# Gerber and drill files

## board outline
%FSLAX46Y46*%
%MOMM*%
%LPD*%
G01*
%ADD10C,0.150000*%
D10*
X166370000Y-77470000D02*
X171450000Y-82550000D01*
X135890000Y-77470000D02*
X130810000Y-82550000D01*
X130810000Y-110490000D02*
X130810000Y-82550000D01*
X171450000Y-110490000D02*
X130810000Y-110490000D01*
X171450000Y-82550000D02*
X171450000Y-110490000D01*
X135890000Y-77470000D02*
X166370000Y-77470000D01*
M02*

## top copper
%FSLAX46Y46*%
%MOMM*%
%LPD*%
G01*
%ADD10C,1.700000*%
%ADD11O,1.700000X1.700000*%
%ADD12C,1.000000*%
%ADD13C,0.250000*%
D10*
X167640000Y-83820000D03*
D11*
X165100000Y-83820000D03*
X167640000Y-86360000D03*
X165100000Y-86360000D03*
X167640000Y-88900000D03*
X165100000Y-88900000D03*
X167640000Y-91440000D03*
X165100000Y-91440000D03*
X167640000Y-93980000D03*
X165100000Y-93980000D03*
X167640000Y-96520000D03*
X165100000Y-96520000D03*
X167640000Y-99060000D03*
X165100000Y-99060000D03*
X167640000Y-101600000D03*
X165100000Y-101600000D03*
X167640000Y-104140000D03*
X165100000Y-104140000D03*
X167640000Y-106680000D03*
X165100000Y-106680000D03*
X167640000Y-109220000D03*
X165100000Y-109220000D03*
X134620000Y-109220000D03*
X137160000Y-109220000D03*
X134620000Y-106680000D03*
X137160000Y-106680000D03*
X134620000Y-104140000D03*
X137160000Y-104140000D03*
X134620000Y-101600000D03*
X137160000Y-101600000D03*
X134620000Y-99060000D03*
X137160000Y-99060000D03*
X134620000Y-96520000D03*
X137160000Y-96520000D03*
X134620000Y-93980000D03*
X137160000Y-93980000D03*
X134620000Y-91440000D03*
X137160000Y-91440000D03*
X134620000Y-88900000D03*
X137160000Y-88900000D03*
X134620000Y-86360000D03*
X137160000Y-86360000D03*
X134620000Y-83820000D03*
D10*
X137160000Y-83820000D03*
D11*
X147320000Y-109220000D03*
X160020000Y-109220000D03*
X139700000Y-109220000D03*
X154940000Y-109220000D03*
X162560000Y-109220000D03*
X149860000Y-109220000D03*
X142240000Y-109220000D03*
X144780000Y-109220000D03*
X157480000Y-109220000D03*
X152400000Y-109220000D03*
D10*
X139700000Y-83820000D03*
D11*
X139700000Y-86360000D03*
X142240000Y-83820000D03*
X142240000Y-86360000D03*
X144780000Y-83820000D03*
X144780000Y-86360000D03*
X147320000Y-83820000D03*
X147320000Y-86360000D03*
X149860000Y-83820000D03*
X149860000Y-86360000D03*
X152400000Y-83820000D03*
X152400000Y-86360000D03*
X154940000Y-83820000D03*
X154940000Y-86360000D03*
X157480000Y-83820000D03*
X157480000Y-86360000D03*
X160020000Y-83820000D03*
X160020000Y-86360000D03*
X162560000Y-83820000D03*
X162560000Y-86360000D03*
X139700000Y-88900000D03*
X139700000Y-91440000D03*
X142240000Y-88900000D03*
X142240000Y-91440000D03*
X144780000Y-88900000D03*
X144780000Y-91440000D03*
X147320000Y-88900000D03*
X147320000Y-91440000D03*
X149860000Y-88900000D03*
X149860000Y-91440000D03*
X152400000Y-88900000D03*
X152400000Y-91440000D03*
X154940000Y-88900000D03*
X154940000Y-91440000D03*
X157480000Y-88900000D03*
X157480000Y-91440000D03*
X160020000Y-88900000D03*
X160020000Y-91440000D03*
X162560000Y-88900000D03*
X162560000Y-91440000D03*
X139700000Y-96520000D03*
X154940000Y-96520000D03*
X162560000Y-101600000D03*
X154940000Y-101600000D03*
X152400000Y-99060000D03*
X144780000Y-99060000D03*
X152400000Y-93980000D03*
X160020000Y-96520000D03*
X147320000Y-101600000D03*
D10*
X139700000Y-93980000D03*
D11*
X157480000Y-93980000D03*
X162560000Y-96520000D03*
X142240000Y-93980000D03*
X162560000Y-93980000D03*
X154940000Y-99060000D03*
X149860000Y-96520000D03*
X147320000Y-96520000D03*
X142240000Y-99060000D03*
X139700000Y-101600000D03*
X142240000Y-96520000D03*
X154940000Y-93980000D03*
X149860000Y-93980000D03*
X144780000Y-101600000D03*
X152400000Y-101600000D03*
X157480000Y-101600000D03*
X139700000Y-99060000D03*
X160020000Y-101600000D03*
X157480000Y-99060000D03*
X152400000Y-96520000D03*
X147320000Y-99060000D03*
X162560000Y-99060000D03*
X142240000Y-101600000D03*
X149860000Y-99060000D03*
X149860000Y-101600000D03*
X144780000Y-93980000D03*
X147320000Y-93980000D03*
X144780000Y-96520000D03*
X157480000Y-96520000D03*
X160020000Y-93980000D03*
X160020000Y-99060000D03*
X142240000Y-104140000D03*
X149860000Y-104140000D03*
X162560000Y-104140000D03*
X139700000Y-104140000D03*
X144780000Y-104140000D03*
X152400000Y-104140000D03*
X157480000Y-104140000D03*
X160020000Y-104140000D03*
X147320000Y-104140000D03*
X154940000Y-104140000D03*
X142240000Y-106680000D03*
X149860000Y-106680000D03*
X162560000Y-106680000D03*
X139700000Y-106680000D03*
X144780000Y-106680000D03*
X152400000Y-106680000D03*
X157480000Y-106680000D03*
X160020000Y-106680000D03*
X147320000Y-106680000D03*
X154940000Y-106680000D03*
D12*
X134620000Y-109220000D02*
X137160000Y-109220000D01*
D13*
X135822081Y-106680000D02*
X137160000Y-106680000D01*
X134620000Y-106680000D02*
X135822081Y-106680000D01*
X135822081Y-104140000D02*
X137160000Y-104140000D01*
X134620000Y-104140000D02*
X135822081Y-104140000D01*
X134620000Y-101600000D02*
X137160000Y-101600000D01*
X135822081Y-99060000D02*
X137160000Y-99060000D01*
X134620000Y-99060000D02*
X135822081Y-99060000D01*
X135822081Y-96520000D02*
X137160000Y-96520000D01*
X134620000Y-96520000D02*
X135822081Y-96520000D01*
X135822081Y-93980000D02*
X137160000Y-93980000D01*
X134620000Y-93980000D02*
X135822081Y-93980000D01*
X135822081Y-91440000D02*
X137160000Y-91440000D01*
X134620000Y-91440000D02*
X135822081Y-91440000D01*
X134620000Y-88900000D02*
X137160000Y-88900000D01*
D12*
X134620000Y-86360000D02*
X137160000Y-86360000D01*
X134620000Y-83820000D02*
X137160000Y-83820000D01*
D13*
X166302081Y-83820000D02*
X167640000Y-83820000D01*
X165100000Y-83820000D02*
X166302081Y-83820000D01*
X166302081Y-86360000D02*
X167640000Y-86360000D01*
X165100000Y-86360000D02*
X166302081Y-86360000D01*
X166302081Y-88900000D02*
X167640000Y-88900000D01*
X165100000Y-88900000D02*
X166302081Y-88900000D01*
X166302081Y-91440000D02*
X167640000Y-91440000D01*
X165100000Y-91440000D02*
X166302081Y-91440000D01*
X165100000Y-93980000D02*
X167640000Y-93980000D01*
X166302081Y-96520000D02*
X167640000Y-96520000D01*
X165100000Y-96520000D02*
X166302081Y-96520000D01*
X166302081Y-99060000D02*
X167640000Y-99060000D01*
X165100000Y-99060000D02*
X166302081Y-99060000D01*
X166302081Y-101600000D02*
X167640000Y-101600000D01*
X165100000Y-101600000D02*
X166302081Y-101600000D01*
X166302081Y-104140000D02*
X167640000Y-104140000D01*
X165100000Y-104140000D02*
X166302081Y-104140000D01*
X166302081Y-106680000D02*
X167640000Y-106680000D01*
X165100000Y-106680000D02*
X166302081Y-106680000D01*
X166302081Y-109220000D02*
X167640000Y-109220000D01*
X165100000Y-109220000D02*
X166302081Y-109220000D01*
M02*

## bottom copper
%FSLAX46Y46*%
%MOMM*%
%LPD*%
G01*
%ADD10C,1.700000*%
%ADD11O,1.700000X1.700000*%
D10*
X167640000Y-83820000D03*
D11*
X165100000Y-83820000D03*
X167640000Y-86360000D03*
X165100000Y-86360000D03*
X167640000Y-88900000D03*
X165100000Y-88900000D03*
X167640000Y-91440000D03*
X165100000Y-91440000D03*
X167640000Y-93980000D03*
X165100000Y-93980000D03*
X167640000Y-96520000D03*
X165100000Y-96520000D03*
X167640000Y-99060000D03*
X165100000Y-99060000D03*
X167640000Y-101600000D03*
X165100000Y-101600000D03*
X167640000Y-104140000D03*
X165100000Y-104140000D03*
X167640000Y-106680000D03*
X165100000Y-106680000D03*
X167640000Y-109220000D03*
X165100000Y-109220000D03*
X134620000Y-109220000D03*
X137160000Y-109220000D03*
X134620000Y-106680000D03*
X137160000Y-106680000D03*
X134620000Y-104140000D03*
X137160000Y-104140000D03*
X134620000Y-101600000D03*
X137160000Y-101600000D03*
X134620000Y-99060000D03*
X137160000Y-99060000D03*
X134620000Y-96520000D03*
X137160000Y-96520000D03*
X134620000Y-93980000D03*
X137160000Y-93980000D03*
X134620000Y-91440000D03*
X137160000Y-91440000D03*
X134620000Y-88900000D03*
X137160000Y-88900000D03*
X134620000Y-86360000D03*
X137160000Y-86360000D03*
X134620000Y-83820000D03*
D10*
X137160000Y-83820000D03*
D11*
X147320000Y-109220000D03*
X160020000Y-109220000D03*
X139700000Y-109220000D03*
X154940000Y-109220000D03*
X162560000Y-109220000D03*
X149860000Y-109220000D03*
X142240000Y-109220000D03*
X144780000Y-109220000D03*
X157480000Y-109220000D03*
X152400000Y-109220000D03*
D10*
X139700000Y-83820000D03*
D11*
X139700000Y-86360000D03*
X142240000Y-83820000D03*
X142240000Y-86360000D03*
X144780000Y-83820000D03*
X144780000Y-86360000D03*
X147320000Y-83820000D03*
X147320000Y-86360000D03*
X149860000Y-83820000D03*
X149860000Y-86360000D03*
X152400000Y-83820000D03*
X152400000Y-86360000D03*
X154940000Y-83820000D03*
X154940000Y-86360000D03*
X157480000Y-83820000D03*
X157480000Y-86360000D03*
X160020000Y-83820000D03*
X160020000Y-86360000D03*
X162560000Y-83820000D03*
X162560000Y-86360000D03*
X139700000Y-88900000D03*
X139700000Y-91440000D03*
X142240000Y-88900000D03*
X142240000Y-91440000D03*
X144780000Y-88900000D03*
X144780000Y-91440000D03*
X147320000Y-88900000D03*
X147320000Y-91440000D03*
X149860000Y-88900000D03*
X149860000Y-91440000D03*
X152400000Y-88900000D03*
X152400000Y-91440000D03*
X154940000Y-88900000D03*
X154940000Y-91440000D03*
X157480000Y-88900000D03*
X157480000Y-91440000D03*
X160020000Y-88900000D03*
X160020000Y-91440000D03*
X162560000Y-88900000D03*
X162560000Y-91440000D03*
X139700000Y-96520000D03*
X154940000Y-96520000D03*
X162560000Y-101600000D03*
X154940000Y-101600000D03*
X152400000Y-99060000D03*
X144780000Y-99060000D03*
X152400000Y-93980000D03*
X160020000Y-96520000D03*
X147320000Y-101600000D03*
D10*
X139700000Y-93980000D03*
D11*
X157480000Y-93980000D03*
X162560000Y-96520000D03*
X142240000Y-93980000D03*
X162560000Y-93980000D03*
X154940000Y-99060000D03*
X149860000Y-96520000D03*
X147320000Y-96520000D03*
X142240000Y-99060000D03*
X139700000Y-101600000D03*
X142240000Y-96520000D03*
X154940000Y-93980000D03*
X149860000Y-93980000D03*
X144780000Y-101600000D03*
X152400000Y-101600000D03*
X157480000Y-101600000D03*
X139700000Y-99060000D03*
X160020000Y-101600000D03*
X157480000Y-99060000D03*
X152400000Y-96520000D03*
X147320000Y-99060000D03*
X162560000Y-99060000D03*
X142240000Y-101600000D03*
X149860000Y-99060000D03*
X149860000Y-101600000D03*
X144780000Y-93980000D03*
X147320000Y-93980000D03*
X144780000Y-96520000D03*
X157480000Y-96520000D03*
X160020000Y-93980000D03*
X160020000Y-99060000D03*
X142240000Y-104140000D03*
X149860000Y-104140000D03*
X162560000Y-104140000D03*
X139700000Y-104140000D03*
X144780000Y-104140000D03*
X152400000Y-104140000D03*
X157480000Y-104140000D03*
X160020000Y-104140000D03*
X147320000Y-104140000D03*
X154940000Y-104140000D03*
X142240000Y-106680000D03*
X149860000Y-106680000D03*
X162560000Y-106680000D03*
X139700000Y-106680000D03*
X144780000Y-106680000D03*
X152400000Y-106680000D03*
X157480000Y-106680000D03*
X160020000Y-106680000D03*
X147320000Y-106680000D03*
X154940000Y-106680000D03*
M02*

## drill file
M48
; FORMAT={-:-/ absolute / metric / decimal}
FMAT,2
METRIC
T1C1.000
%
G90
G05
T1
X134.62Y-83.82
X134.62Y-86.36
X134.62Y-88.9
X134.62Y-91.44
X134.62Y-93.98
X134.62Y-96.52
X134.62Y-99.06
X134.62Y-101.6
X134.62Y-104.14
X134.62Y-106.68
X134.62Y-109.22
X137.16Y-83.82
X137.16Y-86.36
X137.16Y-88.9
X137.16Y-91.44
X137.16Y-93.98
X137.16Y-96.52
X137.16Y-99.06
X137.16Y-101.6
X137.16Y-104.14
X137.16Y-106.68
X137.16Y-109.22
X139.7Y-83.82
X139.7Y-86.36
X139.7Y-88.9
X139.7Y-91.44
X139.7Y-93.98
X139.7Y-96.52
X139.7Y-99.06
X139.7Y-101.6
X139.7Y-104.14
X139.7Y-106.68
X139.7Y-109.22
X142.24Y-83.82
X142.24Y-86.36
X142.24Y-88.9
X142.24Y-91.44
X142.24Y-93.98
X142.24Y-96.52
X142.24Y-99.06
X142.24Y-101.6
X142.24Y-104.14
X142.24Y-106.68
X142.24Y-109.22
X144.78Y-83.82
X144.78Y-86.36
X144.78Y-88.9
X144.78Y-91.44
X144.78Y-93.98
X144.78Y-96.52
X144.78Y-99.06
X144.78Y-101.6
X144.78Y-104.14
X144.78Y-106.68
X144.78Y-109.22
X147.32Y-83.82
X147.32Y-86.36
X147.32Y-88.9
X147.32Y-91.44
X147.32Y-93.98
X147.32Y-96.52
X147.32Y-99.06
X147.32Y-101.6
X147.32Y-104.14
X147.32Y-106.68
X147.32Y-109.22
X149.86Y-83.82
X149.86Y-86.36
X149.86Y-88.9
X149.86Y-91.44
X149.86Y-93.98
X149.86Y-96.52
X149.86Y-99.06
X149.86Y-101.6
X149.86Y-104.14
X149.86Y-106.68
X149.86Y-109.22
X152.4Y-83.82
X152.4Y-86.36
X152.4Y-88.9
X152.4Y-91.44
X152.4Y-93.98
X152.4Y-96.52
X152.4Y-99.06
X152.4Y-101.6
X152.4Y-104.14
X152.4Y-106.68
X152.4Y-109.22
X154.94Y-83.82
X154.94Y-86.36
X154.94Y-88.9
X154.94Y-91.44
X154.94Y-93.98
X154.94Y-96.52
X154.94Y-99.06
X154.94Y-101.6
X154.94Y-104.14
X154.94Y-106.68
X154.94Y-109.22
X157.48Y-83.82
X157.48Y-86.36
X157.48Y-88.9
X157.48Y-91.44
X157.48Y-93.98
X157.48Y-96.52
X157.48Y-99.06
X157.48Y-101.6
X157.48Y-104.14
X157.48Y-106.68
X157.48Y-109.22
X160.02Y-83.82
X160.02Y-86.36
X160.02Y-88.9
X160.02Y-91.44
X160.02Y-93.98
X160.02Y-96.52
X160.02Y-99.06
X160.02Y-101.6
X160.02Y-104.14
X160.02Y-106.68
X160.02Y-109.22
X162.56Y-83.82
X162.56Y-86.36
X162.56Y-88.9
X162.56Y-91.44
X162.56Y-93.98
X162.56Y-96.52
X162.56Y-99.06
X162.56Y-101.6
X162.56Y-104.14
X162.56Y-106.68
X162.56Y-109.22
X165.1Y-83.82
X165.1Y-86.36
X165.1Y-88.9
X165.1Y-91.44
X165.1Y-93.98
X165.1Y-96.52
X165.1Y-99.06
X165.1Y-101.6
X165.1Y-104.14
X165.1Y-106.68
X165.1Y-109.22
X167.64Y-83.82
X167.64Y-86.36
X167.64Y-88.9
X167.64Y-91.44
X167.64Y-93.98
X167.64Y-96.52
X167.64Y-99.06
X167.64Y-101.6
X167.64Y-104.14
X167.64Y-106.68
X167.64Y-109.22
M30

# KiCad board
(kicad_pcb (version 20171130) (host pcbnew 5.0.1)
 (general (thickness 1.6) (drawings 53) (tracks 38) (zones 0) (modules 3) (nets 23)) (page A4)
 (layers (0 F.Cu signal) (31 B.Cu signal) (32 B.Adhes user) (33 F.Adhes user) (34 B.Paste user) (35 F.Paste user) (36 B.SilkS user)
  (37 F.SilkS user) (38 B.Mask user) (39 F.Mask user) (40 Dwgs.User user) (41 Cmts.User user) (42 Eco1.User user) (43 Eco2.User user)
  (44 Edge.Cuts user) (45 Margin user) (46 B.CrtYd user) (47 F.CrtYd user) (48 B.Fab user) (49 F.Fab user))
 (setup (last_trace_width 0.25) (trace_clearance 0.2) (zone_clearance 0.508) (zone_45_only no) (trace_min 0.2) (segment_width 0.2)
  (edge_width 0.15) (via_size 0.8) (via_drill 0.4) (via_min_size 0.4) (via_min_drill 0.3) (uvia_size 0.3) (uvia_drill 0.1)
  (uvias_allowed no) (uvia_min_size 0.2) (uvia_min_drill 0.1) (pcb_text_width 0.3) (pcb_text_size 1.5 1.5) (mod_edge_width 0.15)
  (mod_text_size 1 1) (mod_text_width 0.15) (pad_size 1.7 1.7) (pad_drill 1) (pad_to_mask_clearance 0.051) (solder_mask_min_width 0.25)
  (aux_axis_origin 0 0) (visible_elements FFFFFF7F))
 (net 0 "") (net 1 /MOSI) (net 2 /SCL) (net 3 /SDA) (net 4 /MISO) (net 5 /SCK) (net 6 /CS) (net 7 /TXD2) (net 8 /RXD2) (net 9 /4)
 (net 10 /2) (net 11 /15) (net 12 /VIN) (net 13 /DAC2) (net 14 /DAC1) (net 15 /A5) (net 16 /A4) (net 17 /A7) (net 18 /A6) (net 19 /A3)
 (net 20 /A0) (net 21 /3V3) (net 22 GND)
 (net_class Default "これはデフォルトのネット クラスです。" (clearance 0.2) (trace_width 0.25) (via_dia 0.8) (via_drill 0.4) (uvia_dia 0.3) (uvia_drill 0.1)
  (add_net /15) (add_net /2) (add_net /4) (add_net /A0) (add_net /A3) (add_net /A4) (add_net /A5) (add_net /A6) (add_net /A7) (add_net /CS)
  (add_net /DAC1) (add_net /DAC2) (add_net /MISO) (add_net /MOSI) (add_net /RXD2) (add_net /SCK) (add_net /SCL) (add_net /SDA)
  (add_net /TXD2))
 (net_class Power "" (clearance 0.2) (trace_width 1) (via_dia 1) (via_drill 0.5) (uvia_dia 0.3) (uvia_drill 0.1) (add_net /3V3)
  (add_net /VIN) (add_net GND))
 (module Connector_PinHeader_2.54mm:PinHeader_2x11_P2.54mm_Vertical (layer B.Cu) (at 167.64 83.82 180)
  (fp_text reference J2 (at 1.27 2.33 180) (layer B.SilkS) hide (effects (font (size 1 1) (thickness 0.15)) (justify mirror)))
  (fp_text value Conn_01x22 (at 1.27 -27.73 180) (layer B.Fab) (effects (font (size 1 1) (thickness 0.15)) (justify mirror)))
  (pad 1 thru_hole circle (at 0 0 180) (size 1.7 1.7) (drill 1) (layers *.Cu *.Mask) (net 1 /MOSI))
  (pad 2 thru_hole oval (at 2.54 0 180) (size 1.7 1.7) (drill 1) (layers *.Cu *.Mask) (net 1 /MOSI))
  (pad 3 thru_hole oval (at 0 -2.54 180) (size 1.7 1.7) (drill 1) (layers *.Cu *.Mask) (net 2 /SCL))
  (pad 4 thru_hole oval (at 2.54 -2.54 180) (size 1.7 1.7) (drill 1) (layers *.Cu *.Mask) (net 2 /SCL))
  (pad 5 thru_hole oval (at 0 -5.08 180) (size 1.7 1.7) (drill 1) (layers *.Cu *.Mask) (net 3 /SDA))
  (pad 6 thru_hole oval (at 2.54 -5.08 180) (size 1.7 1.7) (drill 1) (layers *.Cu *.Mask) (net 3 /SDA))
  (pad 7 thru_hole oval (at 0 -7.62 180) (size 1.7 1.7) (drill 1) (layers *.Cu *.Mask) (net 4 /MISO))
  (pad 8 thru_hole oval (at 2.54 -7.62 180) (size 1.7 1.7) (drill 1) (layers *.Cu *.Mask) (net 4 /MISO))
  (pad 9 thru_hole oval (at 0 -10.16 180) (size 1.7 1.7) (drill 1) (layers *.Cu *.Mask) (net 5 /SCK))
  (pad 10 thru_hole oval (at 2.54 -10.16 180) (size 1.7 1.7) (drill 1) (layers *.Cu *.Mask) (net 5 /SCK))
  (pad 11 thru_hole oval (at 0 -12.7 180) (size 1.7 1.7) (drill 1) (layers *.Cu *.Mask) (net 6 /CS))
  (pad 12 thru_hole oval (at 2.54 -12.7 180) (size 1.7 1.7) (drill 1) (layers *.Cu *.Mask) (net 6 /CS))
  (pad 13 thru_hole oval (at 0 -15.24 180) (size 1.7 1.7) (drill 1) (layers *.Cu *.Mask) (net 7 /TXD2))
  (pad 14 thru_hole oval (at 2.54 -15.24 180) (size 1.7 1.7) (drill 1) (layers *.Cu *.Mask) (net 7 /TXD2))
  (pad 15 thru_hole oval (at 0 -17.78 180) (size 1.7 1.7) (drill 1) (layers *.Cu *.Mask) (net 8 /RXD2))
  (pad 16 thru_hole oval (at 2.54 -17.78 180) (size 1.7 1.7) (drill 1) (layers *.Cu *.Mask) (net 8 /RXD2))
  (pad 17 thru_hole oval (at 0 -20.32 180) (size 1.7 1.7) (drill 1) (layers *.Cu *.Mask) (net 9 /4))
  (pad 18 thru_hole oval (at 2.54 -20.32 180) (size 1.7 1.7) (drill 1) (layers *.Cu *.Mask) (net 9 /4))
  (pad 19 thru_hole oval (at 0 -22.86 180) (size 1.7 1.7) (drill 1) (layers *.Cu *.Mask) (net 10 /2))
  (pad 20 thru_hole oval (at 2.54 -22.86 180) (size 1.7 1.7) (drill 1) (layers *.Cu *.Mask) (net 10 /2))
  (pad 21 thru_hole oval (at 0 -25.4 180) (size 1.7 1.7) (drill 1) (layers *.Cu *.Mask) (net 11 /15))
  (pad 22 thru_hole oval (at 2.54 -25.4 180) (size 1.7 1.7) (drill 1) (layers *.Cu *.Mask) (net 11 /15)))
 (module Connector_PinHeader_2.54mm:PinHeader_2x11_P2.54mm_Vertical (layer B.Cu) (at 137.16 83.82 180)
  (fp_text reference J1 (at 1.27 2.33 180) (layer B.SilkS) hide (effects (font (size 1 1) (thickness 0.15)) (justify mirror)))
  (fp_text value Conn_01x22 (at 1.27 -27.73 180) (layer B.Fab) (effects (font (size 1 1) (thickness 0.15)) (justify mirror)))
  (pad 22 thru_hole oval (at 2.54 -25.4 180) (size 1.7 1.7) (drill 1) (layers *.Cu *.Mask) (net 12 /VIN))
  (pad 21 thru_hole oval (at 0 -25.4 180) (size 1.7 1.7) (drill 1) (layers *.Cu *.Mask) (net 12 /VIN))
  (pad 20 thru_hole oval (at 2.54 -22.86 180) (size 1.7 1.7) (drill 1) (layers *.Cu *.Mask) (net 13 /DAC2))
  (pad 19 thru_hole oval (at 0 -22.86 180) (size 1.7 1.7) (drill 1) (layers *.Cu *.Mask) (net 13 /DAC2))
  (pad 18 thru_hole oval (at 2.54 -20.32 180) (size 1.7 1.7) (drill 1) (layers *.Cu *.Mask) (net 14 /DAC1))
  (pad 17 thru_hole oval (at 0 -20.32 180) (size 1.7 1.7) (drill 1) (layers *.Cu *.Mask) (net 14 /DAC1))
  (pad 16 thru_hole oval (at 2.54 -17.78 180) (size 1.7 1.7) (drill 1) (layers *.Cu *.Mask) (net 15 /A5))
  (pad 15 thru_hole oval (at 0 -17.78 180) (size 1.7 1.7) (drill 1) (layers *.Cu *.Mask) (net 15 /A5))
  (pad 14 thru_hole oval (at 2.54 -15.24 180) (size 1.7 1.7) (drill 1) (layers *.Cu *.Mask) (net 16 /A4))
  (pad 13 thru_hole oval (at 0 -15.24 180) (size 1.7 1.7) (drill 1) (layers *.Cu *.Mask) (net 16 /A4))
  (pad 12 thru_hole oval (at 2.54 -12.7 180) (size 1.7 1.7) (drill 1) (layers *.Cu *.Mask) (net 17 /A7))
  (pad 11 thru_hole oval (at 0 -12.7 180) (size 1.7 1.7) (drill 1) (layers *.Cu *.Mask) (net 17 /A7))
  (pad 10 thru_hole oval (at 2.54 -10.16 180) (size 1.7 1.7) (drill 1) (layers *.Cu *.Mask) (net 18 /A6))
  (pad 9 thru_hole oval (at 0 -10.16 180) (size 1.7 1.7) (drill 1) (layers *.Cu *.Mask) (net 18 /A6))
  (pad 8 thru_hole oval (at 2.54 -7.62 180) (size 1.7 1.7) (drill 1) (layers *.Cu *.Mask) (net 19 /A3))
  (pad 7 thru_hole oval (at 0 -7.62 180) (size 1.7 1.7) (drill 1) (layers *.Cu *.Mask) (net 19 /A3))
  (pad 6 thru_hole oval (at 2.54 -5.08 180) (size 1.7 1.7) (drill 1) (layers *.Cu *.Mask) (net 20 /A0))
  (pad 5 thru_hole oval (at 0 -5.08 180) (size 1.7 1.7) (drill 1) (layers *.Cu *.Mask) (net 20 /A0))
  (pad 4 thru_hole oval (at 2.54 -2.54 180) (size 1.7 1.7) (drill 1) (layers *.Cu *.Mask) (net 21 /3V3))
  (pad 3 thru_hole oval (at 0 -2.54 180) (size 1.7 1.7) (drill 1) (layers *.Cu *.Mask) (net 21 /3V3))
  (pad 2 thru_hole oval (at 2.54 0 180) (size 1.7 1.7) (drill 1) (layers *.Cu *.Mask) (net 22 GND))
  (pad 1 thru_hole circle (at 0 0 180) (size 1.7 1.7) (drill 1) (layers *.Cu *.Mask) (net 22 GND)))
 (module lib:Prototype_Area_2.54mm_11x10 (layer F.Cu) (at 139.7 83.82 90)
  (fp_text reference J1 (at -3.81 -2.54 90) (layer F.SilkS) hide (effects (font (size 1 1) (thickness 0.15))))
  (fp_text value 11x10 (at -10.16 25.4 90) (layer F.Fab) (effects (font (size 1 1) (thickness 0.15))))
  (pad 34 thru_hole oval (at -25.4 7.62 90) (size 1.7 1.7) (drill 1) (layers *.Cu *.Mask))
  (pad 99 thru_hole oval (at -25.4 20.32 90) (size 1.7 1.7) (drill 1) (layers *.Cu *.Mask))
  (pad 11 thru_hole oval (at -25.4 0 90) (size 1.7 1.7) (drill 1) (layers *.Cu *.Mask))
  (pad 77 thru_hole oval (at -25.4 15.24 90) (size 1.7 1.7) (drill 1) (layers *.Cu *.Mask))
  (pad 100 thru_hole oval (at -25.4 22.86 90) (size 1.7 1.7) (drill 1) (layers *.Cu *.Mask))
  (pad 55 thru_hole oval (at -25.4 10.16 90) (size 1.7 1.7) (drill 1) (layers *.Cu *.Mask))
  (pad 12 thru_hole oval (at -25.4 2.54 90) (size 1.7 1.7) (drill 1) (layers *.Cu *.Mask))
  (pad 33 thru_hole oval (at -25.4 5.08 90) (size 1.7 1.7) (drill 1) (layers *.Cu *.Mask))
  (pad 78 thru_hole oval (at -25.4 17.78 90) (size 1.7 1.7) (drill 1) (layers *.Cu *.Mask))
  (pad 56 thru_hole oval (at -25.4 12.7 90) (size 1.7 1.7) (drill 1) (layers *.Cu *.Mask))
  (pad 1 thru_hole circle (at 0 0 90) (size 1.7 1.7) (drill 1) (layers *.Cu *.Mask))
  (pad 2 thru_hole oval (at -2.54 0 90) (size 1.7 1.7) (drill 1) (layers *.Cu *.Mask))
  (pad 22 thru_hole oval (at 0 2.54 90) (size 1.7 1.7) (drill 1) (layers *.Cu *.Mask))
  (pad 21 thru_hole oval (at -2.54 2.54 90) (size 1.7 1.7) (drill 1) (layers *.Cu *.Mask))
  (pad 23 thru_hole oval (at 0 5.08 90) (size 1.7 1.7) (drill 1) (layers *.Cu *.Mask))
  (pad 24 thru_hole oval (at -2.54 5.08 90) (size 1.7 1.7) (drill 1) (layers *.Cu *.Mask))
  (pad 44 thru_hole oval (at 0 7.62 90) (size 1.7 1.7) (drill 1) (layers *.Cu *.Mask))
  (pad 43 thru_hole oval (at -2.54 7.62 90) (size 1.7 1.7) (drill 1) (layers *.Cu *.Mask))
  (pad 45 thru_hole oval (at 0 10.16 90) (size 1.7 1.7) (drill 1) (layers *.Cu *.Mask))
  (pad 46 thru_hole oval (at -2.54 10.16 90) (size 1.7 1.7) (drill 1) (layers *.Cu *.Mask))
  (pad 66 thru_hole oval (at 0 12.7 90) (size 1.7 1.7) (drill 1) (layers *.Cu *.Mask))
  (pad 65 thru_hole oval (at -2.54 12.7 90) (size 1.7 1.7) (drill 1) (layers *.Cu *.Mask))
  (pad 67 thru_hole oval (at 0 15.24 90) (size 1.7 1.7) (drill 1) (layers *.Cu *.Mask))
  (pad 68 thru_hole oval (at -2.54 15.24 90) (size 1.7 1.7) (drill 1) (layers *.Cu *.Mask))
  (pad 88 thru_hole oval (at 0 17.78 90) (size 1.7 1.7) (drill 1) (layers *.Cu *.Mask))
  (pad 87 thru_hole oval (at -2.54 17.78 90) (size 1.7 1.7) (drill 1) (layers *.Cu *.Mask))
  (pad 89 thru_hole oval (at 0 20.32 90) (size 1.7 1.7) (drill 1) (layers *.Cu *.Mask))
  (pad 90 thru_hole oval (at -2.54 20.32 90) (size 1.7 1.7) (drill 1) (layers *.Cu *.Mask))
  (pad 110 thru_hole oval (at 0 22.86 90) (size 1.7 1.7) (drill 1) (layers *.Cu *.Mask))
  (pad 109 thru_hole oval (at -2.54 22.86 90) (size 1.7 1.7) (drill 1) (layers *.Cu *.Mask))
  (pad 3 thru_hole oval (at -5.08 0 90) (size 1.7 1.7) (drill 1) (layers *.Cu *.Mask))
  (pad 4 thru_hole oval (at -7.62 0 90) (size 1.7 1.7) (drill 1) (layers *.Cu *.Mask))
  (pad 20 thru_hole oval (at -5.08 2.54 90) (size 1.7 1.7) (drill 1) (layers *.Cu *.Mask))
  (pad 19 thru_hole oval (at -7.62 2.54 90) (size 1.7 1.7) (drill 1) (layers *.Cu *.Mask))
  (pad 25 thru_hole oval (at -5.08 5.08 90) (size 1.7 1.7) (drill 1) (layers *.Cu *.Mask))
  (pad 26 thru_hole oval (at -7.62 5.08 90) (size 1.7 1.7) (drill 1) (layers *.Cu *.Mask))
  (pad 42 thru_hole oval (at -5.08 7.62 90) (size 1.7 1.7) (drill 1) (layers *.Cu *.Mask))
  (pad 41 thru_hole oval (at -7.62 7.62 90) (size 1.7 1.7) (drill 1) (layers *.Cu *.Mask))
  (pad 47 thru_hole oval (at -5.08 10.16 90) (size 1.7 1.7) (drill 1) (layers *.Cu *.Mask))
  (pad 48 thru_hole oval (at -7.62 10.16 90) (size 1.7 1.7) (drill 1) (layers *.Cu *.Mask))
  (pad 64 thru_hole oval (at -5.08 12.7 90) (size 1.7 1.7) (drill 1) (layers *.Cu *.Mask))
  (pad 63 thru_hole oval (at -7.62 12.7 90) (size 1.7 1.7) (drill 1) (layers *.Cu *.Mask))
  (pad 69 thru_hole oval (at -5.08 15.24 90) (size 1.7 1.7) (drill 1) (layers *.Cu *.Mask))
  (pad 70 thru_hole oval (at -7.62 15.24 90) (size 1.7 1.7) (drill 1) (layers *.Cu *.Mask))
  (pad 86 thru_hole oval (at -5.08 17.78 90) (size 1.7 1.7) (drill 1) (layers *.Cu *.Mask))
  (pad 85 thru_hole oval (at -7.62 17.78 90) (size 1.7 1.7) (drill 1) (layers *.Cu *.Mask))
  (pad 91 thru_hole oval (at -5.08 20.32 90) (size 1.7 1.7) (drill 1) (layers *.Cu *.Mask))
  (pad 92 thru_hole oval (at -7.62 20.32 90) (size 1.7 1.7) (drill 1) (layers *.Cu *.Mask))
  (pad 108 thru_hole oval (at -5.08 22.86 90) (size 1.7 1.7) (drill 1) (layers *.Cu *.Mask))
  (pad 107 thru_hole oval (at -7.62 22.86 90) (size 1.7 1.7) (drill 1) (layers *.Cu *.Mask))
  (pad 6 thru_hole oval (at -12.7 0 90) (size 1.7 1.7) (drill 1) (layers *.Cu *.Mask))
  (pad 72 thru_hole oval (at -12.7 15.24 90) (size 1.7 1.7) (drill 1) (layers *.Cu *.Mask))
  (pad 103 thru_hole oval (at -17.78 22.86 90) (size 1.7 1.7) (drill 1) (layers *.Cu *.Mask))
  (pad 74 thru_hole oval (at -17.78 15.24 90) (size 1.7 1.7) (drill 1) (layers *.Cu *.Mask))
  (pad 60 thru_hole oval (at -15.24 12.7 90) (size 1.7 1.7) (drill 1) (layers *.Cu *.Mask))
  (pad 29 thru_hole oval (at -15.24 5.08 90) (size 1.7 1.7) (drill 1) (layers *.Cu *.Mask))
  (pad 62 thru_hole oval (at -10.16 12.7 90) (size 1.7 1.7) (drill 1) (layers *.Cu *.Mask))
  (pad 94 thru_hole oval (at -12.7 20.32 90) (size 1.7 1.7) (drill 1) (layers *.Cu *.Mask))
  (pad 37 thru_hole oval (at -17.78 7.62 90) (size 1.7 1.7) (drill 1) (layers *.Cu *.Mask))
  (pad 5 thru_hole circle (at -10.16 0 90) (size 1.7 1.7) (drill 1) (layers *.Cu *.Mask))
  (pad 84 thru_hole oval (at -10.16 17.78 90) (size 1.7 1.7) (drill 1) (layers *.Cu *.Mask))
  (pad 105 thru_hole oval (at -12.7 22.86 90) (size 1.7 1.7) (drill 1) (layers *.Cu *.Mask))
  (pad 18 thru_hole oval (at -10.16 2.54 90) (size 1.7 1.7) (drill 1) (layers *.Cu *.Mask))
  (pad 106 thru_hole oval (at -10.16 22.86 90) (size 1.7 1.7) (drill 1) (layers *.Cu *.Mask))
  (pad 73 thru_hole oval (at -15.24 15.24 90) (size 1.7 1.7) (drill 1) (layers *.Cu *.Mask))
  (pad 50 thru_hole oval (at -12.7 10.16 90) (size 1.7 1.7) (drill 1) (layers *.Cu *.Mask))
  (pad 39 thru_hole oval (at -12.7 7.62 90) (size 1.7 1.7) (drill 1) (layers *.Cu *.Mask))
  (pad 16 thru_hole oval (at -15.24 2.54 90) (size 1.7 1.7) (drill 1) (layers *.Cu *.Mask))
  (pad 8 thru_hole oval (at -17.78 0 90) (size 1.7 1.7) (drill 1) (layers *.Cu *.Mask))
  (pad 17 thru_hole oval (at -12.7 2.54 90) (size 1.7 1.7) (drill 1) (layers *.Cu *.Mask))
  (pad 71 thru_hole oval (at -10.16 15.24 90) (size 1.7 1.7) (drill 1) (layers *.Cu *.Mask))
  (pad 49 thru_hole oval (at -10.16 10.16 90) (size 1.7 1.7) (drill 1) (layers *.Cu *.Mask))
  (pad 30 thru_hole oval (at -17.78 5.08 90) (size 1.7 1.7) (drill 1) (layers *.Cu *.Mask))
  (pad 59 thru_hole oval (at -17.78 12.7 90) (size 1.7 1.7) (drill 1) (layers *.Cu *.Mask))
  (pad 81 thru_hole oval (at -17.78 17.78 90) (size 1.7 1.7) (drill 1) (layers *.Cu *.Mask))
  (pad 7 thru_hole oval (at -15.24 0 90) (size 1.7 1.7) (drill 1) (layers *.Cu *.Mask))
  (pad 96 thru_hole oval (at -17.78 20.32 90) (size 1.7 1.7) (drill 1) (layers *.Cu *.Mask))
  (pad 82 thru_hole oval (at -15.24 17.78 90) (size 1.7 1.7) (drill 1) (layers *.Cu *.Mask))
  (pad 61 thru_hole oval (at -12.7 12.7 90) (size 1.7 1.7) (drill 1) (layers *.Cu *.Mask))
  (pad 38 thru_hole oval (at -15.24 7.62 90) (size 1.7 1.7) (drill 1) (layers *.Cu *.Mask))
  (pad 104 thru_hole oval (at -15.24 22.86 90) (size 1.7 1.7) (drill 1) (layers *.Cu *.Mask))
  (pad 15 thru_hole oval (at -17.78 2.54 90) (size 1.7 1.7) (drill 1) (layers *.Cu *.Mask))
  (pad 51 thru_hole oval (at -15.24 10.16 90) (size 1.7 1.7) (drill 1) (layers *.Cu *.Mask))
  (pad 52 thru_hole oval (at -17.78 10.16 90) (size 1.7 1.7) (drill 1) (layers *.Cu *.Mask))
  (pad 27 thru_hole oval (at -10.16 5.08 90) (size 1.7 1.7) (drill 1) (layers *.Cu *.Mask))
  (pad 40 thru_hole oval (at -10.16 7.62 90) (size 1.7 1.7) (drill 1) (layers *.Cu *.Mask))
  (pad 28 thru_hole oval (at -12.7 5.08 90) (size 1.7 1.7) (drill 1) (layers *.Cu *.Mask))
  (pad 83 thru_hole oval (at -12.7 17.78 90) (size 1.7 1.7) (drill 1) (layers *.Cu *.Mask))
  (pad 93 thru_hole oval (at -10.16 20.32 90) (size 1.7 1.7) (drill 1) (layers *.Cu *.Mask))
  (pad 95 thru_hole oval (at -15.24 20.32 90) (size 1.7 1.7) (drill 1) (layers *.Cu *.Mask))
  (pad 14 thru_hole oval (at -20.32 2.54 90) (size 1.7 1.7) (drill 1) (layers *.Cu *.Mask))
  (pad 53 thru_hole oval (at -20.32 10.16 90) (size 1.7 1.7) (drill 1) (layers *.Cu *.Mask))
  (pad 102 thru_hole oval (at -20.32 22.86 90) (size 1.7 1.7) (drill 1) (layers *.Cu *.Mask))
  (pad 9 thru_hole oval (at -20.32 0 90) (size 1.7 1.7) (drill 1) (layers *.Cu *.Mask))
  (pad 31 thru_hole oval (at -20.32 5.08 90) (size 1.7 1.7) (drill 1) (layers *.Cu *.Mask))
  (pad 58 thru_hole oval (at -20.32 12.7 90) (size 1.7 1.7) (drill 1) (layers *.Cu *.Mask))
  (pad 80 thru_hole oval (at -20.32 17.78 90) (size 1.7 1.7) (drill 1) (layers *.Cu *.Mask))
  (pad 97 thru_hole oval (at -20.32 20.32 90) (size 1.7 1.7) (drill 1) (layers *.Cu *.Mask))
  (pad 36 thru_hole oval (at -20.32 7.62 90) (size 1.7 1.7) (drill 1) (layers *.Cu *.Mask))
  (pad 75 thru_hole oval (at -20.32 15.24 90) (size 1.7 1.7) (drill 1) (layers *.Cu *.Mask))
  (pad 13 thru_hole oval (at -22.86 2.54 90) (size 1.7 1.7) (drill 1) (layers *.Cu *.Mask))
  (pad 54 thru_hole oval (at -22.86 10.16 90) (size 1.7 1.7) (drill 1) (layers *.Cu *.Mask))
  (pad 101 thru_hole oval (at -22.86 22.86 90) (size 1.7 1.7) (drill 1) (layers *.Cu *.Mask))
  (pad 10 thru_hole oval (at -22.86 0 90) (size 1.7 1.7) (drill 1) (layers *.Cu *.Mask))
  (pad 32 thru_hole oval (at -22.86 5.08 90) (size 1.7 1.7) (drill 1) (layers *.Cu *.Mask))
  (pad 57 thru_hole oval (at -22.86 12.7 90) (size 1.7 1.7) (drill 1) (layers *.Cu *.Mask))
  (pad 79 thru_hole oval (at -22.86 17.78 90) (size 1.7 1.7) (drill 1) (layers *.Cu *.Mask))
  (pad 98 thru_hole oval (at -22.86 20.32 90) (size 1.7 1.7) (drill 1) (layers *.Cu *.Mask))
  (pad 35 thru_hole oval (at -22.86 7.62 90) (size 1.7 1.7) (drill 1) (layers *.Cu *.Mask))
  (pad 76 thru_hole oval (at -22.86 15.24 90) (size 1.7 1.7) (drill 1) (layers *.Cu *.Mask)))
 (gr_line (start 166.37 77.47) (end 171.45 82.55) (layer Edge.Cuts) (width 0.15))
 (gr_line (start 135.89 77.47) (end 130.81 82.55) (layer Edge.Cuts) (width 0.15))
 (gr_line (start 130.81 110.49) (end 130.81 82.55) (layer Edge.Cuts) (width 0.15))
 (gr_line (start 171.45 110.49) (end 130.81 110.49) (layer Edge.Cuts) (width 0.15))
 (gr_line (start 171.45 82.55) (end 171.45 110.49) (layer Edge.Cuts) (width 0.15))
 (gr_line (start 135.89 77.47) (end 166.37 77.47) (layer Edge.Cuts) (width 0.15))
 (segment (start 134.62 109.22) (end 137.16 109.22) (width 1) (layer F.Cu) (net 12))
 (segment (start 135.822081 106.68) (end 137.16 106.68) (width 0.25) (layer F.Cu) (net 13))
 (segment (start 134.62 106.68) (end 135.822081 106.68) (width 0.25) (layer F.Cu) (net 13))
 (segment (start 135.822081 104.14) (end 137.16 104.14) (width 0.25) (layer F.Cu) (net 14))
 (segment (start 134.62 104.14) (end 135.822081 104.14) (width 0.25) (layer F.Cu) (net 14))
 (segment (start 134.62 101.6) (end 137.16 101.6) (width 0.25) (layer F.Cu) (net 15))
 (segment (start 135.822081 99.06) (end 137.16 99.06) (width 0.25) (layer F.Cu) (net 16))
 (segment (start 134.62 99.06) (end 135.822081 99.06) (width 0.25) (layer F.Cu) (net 16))
 (segment (start 135.822081 96.52) (end 137.16 96.52) (width 0.25) (layer F.Cu) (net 17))
 (segment (start 134.62 96.52) (end 135.822081 96.52) (width 0.25) (layer F.Cu) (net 17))
 (segment (start 135.822081 93.98) (end 137.16 93.98) (width 0.25) (layer F.Cu) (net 18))
 (segment (start 134.62 93.98) (end 135.822081 93.98) (width 0.25) (layer F.Cu) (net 18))
 (segment (start 135.822081 91.44) (end 137.16 91.44) (width 0.25) (layer F.Cu) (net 19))
 (segment (start 134.62 91.44) (end 135.822081 91.44) (width 0.25) (layer F.Cu) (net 19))
 (segment (start 134.62 88.9) (end 137.16 88.9) (width 0.25) (layer F.Cu) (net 20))
 (segment (start 134.62 86.36) (end 137.16 86.36) (width 1) (layer F.Cu) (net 21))
 (segment (start 134.62 83.82) (end 137.16 83.82) (width 1) (layer F.Cu) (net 22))
 (segment (start 166.302081 83.82) (end 167.64 83.82) (width 0.25) (layer F.Cu) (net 1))
 (segment (start 165.1 83.82) (end 166.302081 83.82) (width 0.25) (layer F.Cu) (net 1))
 (segment (start 166.302081 86.36) (end 167.64 86.36) (width 0.25) (layer F.Cu) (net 2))
 (segment (start 165.1 86.36) (end 166.302081 86.36) (width 0.25) (layer F.Cu) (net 2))
 (segment (start 166.302081 88.9) (end 167.64 88.9) (width 0.25) (layer F.Cu) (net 3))
 (segment (start 165.1 88.9) (end 166.302081 88.9) (width 0.25) (layer F.Cu) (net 3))
 (segment (start 166.302081 91.44) (end 167.64 91.44) (width 0.25) (layer F.Cu) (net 4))
 (segment (start 165.1 91.44) (end 166.302081 91.44) (width 0.25) (layer F.Cu) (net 4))
 (segment (start 165.1 93.98) (end 167.64 93.98) (width 0.25) (layer F.Cu) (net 5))
 (segment (start 166.302081 96.52) (end 167.64 96.52) (width 0.25) (layer F.Cu) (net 6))
 (segment (start 165.1 96.52) (end 166.302081 96.52) (width 0.25) (layer F.Cu) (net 6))
 (segment (start 166.302081 99.06) (end 167.64 99.06) (width 0.25) (layer F.Cu) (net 7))
 (segment (start 165.1 99.06) (end 166.302081 99.06) (width 0.25) (layer F.Cu) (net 7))
 (segment (start 166.302081 101.6) (end 167.64 101.6) (width 0.25) (layer F.Cu) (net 8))
 (segment (start 165.1 101.6) (end 166.302081 101.6) (width 0.25) (layer F.Cu) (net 8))
 (segment (start 166.302081 104.14) (end 167.64 104.14) (width 0.25) (layer F.Cu) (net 9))
 (segment (start 165.1 104.14) (end 166.302081 104.14) (width 0.25) (layer F.Cu) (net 9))
 (segment (start 166.302081 106.68) (end 167.64 106.68) (width 0.25) (layer F.Cu) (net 10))
 (segment (start 165.1 106.68) (end 166.302081 106.68) (width 0.25) (layer F.Cu) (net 10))
 (segment (start 166.302081 109.22) (end 167.64 109.22) (width 0.25) (layer F.Cu) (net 11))
 (segment (start 165.1 109.22) (end 166.302081 109.22) (width 0.25) (layer F.Cu) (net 11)))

